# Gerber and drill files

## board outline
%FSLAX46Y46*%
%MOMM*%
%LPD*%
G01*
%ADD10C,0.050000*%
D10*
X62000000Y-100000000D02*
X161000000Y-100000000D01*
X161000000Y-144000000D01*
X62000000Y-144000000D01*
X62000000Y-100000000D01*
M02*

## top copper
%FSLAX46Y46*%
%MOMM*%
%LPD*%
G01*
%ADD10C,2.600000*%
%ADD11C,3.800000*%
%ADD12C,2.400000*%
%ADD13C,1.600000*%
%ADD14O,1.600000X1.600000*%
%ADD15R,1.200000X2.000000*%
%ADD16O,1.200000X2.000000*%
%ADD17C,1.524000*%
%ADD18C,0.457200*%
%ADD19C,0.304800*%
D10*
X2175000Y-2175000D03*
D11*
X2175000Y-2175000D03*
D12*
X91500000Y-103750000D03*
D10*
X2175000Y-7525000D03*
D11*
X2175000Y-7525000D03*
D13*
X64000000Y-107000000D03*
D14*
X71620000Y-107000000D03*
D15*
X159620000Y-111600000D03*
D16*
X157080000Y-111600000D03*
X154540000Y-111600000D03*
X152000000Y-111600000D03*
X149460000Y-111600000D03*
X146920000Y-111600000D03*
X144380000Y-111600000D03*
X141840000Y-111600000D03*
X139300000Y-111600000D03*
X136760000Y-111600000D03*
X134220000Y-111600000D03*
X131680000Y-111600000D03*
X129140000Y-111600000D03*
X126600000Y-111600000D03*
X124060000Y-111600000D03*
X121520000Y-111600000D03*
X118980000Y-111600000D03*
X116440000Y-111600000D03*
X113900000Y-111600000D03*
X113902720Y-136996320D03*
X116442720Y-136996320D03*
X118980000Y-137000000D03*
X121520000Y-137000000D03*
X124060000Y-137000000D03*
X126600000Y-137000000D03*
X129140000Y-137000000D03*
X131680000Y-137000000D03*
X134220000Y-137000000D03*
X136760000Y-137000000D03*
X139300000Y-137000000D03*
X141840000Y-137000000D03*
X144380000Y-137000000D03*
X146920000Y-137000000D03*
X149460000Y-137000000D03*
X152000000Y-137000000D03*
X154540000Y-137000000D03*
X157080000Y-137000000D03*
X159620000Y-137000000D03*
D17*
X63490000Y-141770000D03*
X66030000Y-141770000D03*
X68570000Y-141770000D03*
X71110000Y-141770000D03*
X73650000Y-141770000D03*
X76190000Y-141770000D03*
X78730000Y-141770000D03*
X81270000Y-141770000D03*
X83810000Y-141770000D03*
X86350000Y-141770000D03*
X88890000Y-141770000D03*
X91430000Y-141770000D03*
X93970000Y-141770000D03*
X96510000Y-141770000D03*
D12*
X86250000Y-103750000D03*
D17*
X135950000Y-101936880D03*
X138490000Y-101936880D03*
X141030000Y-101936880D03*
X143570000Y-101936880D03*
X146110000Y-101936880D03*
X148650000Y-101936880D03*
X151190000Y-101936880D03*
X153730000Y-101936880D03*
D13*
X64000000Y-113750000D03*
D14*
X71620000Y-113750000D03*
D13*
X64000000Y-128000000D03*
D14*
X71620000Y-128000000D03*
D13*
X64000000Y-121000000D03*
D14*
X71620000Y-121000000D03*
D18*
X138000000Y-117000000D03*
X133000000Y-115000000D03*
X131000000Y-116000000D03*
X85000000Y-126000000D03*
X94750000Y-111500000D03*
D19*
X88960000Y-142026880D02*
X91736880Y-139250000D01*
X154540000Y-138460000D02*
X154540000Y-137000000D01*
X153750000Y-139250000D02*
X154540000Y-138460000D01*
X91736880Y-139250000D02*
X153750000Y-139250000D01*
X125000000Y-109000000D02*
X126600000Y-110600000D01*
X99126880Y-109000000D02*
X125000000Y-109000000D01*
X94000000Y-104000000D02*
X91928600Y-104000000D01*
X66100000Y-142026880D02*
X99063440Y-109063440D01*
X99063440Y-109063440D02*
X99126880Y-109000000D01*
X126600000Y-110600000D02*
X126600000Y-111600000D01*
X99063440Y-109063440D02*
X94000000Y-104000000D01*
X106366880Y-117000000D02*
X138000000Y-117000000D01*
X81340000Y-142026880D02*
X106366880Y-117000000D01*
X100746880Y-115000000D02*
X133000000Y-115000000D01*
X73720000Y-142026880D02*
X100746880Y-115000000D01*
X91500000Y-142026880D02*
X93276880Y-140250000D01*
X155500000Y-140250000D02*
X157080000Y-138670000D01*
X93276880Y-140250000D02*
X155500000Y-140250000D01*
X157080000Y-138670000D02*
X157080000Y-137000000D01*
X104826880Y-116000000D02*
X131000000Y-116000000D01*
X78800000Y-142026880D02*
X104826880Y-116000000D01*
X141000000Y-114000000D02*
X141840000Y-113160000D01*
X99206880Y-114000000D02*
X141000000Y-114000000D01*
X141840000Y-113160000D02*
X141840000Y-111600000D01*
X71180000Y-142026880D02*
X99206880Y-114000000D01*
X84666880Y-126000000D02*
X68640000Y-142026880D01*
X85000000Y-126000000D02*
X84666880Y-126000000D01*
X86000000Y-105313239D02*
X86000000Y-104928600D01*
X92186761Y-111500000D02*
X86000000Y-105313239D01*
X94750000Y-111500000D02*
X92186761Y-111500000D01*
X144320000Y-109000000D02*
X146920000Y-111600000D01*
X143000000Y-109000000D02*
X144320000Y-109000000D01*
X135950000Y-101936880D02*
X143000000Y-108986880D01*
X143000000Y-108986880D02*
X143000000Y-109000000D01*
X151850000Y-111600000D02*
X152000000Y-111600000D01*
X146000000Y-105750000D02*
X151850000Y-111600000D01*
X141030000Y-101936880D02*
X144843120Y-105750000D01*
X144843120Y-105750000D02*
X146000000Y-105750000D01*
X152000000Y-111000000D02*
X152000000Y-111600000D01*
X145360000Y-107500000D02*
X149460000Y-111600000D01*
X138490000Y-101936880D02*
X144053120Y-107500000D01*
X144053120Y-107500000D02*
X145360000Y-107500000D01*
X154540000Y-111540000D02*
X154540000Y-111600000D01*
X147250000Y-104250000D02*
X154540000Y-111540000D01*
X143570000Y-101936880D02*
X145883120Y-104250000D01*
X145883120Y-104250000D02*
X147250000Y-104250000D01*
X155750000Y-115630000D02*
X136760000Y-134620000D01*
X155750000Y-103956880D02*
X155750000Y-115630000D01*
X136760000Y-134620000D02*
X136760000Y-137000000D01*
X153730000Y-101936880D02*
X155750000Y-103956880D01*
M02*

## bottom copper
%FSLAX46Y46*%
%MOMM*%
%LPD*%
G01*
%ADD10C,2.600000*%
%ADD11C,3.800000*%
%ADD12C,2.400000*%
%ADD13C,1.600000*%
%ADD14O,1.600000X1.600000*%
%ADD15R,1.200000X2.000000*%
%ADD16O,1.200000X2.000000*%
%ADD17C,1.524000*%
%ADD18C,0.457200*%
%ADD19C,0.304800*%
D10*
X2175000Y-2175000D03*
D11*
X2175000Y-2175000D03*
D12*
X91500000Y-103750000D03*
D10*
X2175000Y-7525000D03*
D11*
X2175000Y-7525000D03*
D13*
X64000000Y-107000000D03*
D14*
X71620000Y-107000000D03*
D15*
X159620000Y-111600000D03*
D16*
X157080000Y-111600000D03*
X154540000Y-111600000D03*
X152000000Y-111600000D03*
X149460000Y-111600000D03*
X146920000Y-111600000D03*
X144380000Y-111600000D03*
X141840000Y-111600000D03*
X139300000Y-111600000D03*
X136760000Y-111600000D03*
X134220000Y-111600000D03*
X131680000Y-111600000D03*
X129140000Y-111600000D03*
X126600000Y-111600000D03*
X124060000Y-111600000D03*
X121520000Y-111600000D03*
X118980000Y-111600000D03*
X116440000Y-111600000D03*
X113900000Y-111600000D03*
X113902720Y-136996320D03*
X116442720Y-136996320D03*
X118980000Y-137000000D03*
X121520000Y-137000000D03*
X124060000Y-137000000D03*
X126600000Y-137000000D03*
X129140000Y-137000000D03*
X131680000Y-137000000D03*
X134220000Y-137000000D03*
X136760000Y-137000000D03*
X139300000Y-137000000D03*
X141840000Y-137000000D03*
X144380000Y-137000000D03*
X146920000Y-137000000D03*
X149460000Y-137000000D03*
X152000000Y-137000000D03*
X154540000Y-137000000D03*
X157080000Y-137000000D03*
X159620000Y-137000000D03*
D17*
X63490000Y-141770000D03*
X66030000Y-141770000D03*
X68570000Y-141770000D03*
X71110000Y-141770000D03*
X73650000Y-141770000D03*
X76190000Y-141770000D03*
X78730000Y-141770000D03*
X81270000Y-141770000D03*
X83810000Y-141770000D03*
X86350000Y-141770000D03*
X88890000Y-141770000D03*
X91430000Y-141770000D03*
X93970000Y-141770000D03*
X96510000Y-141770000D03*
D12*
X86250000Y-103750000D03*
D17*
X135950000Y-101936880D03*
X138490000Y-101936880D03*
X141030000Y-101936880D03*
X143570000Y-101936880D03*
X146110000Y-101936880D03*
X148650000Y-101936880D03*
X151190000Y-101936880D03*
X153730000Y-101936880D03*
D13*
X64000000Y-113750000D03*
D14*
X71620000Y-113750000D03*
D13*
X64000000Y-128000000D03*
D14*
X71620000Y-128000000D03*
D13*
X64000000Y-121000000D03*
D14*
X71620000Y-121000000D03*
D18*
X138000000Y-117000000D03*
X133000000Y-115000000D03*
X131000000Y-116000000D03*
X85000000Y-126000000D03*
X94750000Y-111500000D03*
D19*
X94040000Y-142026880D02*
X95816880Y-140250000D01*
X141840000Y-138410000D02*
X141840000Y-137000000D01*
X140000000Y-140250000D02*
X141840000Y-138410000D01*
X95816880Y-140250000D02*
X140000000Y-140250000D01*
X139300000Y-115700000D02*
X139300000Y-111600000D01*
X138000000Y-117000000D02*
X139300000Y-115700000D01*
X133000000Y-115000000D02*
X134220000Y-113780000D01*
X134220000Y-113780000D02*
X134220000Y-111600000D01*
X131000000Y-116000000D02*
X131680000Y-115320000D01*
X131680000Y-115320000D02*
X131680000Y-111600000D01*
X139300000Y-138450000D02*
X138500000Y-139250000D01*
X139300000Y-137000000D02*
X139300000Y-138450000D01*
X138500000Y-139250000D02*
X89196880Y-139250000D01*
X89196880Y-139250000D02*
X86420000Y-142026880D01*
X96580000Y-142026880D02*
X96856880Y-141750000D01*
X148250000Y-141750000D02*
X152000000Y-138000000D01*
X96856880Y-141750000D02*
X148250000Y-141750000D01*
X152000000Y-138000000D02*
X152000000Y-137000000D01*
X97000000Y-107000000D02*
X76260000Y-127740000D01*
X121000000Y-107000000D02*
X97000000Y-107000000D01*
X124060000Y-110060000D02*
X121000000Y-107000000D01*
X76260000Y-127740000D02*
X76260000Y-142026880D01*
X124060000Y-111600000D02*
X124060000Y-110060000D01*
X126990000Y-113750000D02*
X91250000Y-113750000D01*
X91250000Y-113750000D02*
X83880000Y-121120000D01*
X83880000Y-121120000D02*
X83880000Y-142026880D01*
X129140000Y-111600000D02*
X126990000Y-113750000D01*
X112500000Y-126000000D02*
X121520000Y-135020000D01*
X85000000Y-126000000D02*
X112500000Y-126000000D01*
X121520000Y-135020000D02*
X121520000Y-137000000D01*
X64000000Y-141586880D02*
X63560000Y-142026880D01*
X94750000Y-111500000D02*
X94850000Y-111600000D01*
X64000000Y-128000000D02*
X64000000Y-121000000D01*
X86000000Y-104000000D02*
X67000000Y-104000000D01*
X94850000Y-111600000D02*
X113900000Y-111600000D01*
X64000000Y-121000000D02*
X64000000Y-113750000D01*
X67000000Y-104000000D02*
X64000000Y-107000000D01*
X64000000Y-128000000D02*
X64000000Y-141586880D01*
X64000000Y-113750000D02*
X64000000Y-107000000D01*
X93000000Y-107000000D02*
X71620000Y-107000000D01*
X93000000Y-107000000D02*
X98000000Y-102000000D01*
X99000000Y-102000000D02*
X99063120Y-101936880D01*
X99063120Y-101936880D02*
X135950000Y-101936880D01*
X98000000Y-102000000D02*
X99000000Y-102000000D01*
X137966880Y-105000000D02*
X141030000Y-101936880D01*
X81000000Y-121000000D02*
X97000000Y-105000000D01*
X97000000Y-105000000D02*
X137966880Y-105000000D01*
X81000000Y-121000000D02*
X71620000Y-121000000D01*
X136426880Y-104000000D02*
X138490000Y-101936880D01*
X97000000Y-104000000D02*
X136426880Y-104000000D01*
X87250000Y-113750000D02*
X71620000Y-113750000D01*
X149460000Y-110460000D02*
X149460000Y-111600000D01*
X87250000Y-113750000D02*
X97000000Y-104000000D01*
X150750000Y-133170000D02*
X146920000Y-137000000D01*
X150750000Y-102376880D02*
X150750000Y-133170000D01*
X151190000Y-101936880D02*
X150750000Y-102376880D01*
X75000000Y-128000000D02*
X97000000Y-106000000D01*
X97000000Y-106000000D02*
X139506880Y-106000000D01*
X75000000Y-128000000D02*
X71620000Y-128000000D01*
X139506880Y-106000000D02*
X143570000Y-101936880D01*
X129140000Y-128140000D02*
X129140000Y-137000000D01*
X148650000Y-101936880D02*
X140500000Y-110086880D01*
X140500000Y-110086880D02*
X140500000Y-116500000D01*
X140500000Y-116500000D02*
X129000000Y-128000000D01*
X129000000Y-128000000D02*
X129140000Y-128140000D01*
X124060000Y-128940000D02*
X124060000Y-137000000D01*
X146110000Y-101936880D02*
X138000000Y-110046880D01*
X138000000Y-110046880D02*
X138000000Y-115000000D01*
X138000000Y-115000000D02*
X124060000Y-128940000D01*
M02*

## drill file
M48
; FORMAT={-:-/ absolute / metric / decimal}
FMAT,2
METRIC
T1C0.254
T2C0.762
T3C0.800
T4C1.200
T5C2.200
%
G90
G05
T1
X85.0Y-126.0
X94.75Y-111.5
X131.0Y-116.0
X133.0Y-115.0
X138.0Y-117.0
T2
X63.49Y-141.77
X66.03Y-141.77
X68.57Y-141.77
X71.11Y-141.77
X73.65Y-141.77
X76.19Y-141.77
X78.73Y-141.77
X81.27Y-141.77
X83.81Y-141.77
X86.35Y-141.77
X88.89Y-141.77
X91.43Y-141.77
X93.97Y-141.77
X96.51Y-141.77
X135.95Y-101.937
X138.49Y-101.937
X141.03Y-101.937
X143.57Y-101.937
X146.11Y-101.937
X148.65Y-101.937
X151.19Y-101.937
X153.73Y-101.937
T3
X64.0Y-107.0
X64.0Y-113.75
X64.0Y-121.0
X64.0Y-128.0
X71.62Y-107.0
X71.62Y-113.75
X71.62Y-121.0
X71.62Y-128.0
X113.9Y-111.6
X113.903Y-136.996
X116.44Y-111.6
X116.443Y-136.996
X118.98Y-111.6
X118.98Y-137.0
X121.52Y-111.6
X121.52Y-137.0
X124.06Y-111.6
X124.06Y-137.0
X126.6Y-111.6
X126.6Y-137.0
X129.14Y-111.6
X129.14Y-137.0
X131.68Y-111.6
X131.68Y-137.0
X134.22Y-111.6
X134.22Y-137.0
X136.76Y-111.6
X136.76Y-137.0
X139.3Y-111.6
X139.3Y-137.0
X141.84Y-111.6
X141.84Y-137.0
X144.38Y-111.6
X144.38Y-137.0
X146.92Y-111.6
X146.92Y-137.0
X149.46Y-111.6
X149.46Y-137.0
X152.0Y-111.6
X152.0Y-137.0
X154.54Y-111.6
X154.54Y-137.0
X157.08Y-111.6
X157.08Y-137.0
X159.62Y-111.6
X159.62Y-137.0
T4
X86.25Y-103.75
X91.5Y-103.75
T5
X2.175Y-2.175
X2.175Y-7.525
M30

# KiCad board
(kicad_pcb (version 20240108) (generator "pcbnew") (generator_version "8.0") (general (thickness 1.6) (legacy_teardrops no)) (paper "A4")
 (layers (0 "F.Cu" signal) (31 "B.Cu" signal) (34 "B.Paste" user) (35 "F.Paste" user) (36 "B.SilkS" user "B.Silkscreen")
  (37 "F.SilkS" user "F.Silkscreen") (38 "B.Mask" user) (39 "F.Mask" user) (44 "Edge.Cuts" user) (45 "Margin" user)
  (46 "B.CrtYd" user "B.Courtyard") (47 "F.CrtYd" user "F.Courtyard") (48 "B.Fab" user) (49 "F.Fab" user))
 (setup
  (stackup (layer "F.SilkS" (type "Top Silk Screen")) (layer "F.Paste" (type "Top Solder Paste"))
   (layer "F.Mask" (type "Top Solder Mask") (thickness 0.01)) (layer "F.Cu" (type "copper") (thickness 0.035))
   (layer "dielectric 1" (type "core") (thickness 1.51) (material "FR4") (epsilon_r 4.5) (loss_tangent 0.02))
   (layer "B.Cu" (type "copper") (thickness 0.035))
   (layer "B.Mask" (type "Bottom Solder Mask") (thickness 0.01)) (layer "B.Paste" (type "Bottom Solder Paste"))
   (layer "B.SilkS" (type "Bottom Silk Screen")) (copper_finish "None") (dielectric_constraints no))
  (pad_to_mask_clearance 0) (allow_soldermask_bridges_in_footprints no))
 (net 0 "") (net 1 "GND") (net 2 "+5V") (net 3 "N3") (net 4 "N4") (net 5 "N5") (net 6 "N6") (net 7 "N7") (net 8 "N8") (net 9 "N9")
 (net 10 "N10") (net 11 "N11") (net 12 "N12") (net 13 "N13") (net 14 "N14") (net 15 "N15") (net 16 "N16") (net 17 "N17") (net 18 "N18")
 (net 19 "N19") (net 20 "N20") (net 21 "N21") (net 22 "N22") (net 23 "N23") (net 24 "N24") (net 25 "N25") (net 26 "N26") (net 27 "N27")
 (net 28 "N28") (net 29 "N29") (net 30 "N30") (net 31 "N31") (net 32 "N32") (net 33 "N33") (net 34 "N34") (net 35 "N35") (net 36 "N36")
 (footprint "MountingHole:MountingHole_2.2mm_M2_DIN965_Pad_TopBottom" (layer "F.Cu") (at 2.175 2.175)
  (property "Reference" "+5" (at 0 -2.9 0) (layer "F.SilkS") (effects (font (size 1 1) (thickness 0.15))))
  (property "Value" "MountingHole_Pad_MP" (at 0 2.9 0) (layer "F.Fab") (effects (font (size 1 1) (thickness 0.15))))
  (pad "1" thru_hole circle (at 0 0) (size 2.6 2.6) (drill 2.2) (layers "*.Cu" "*.Mask") (remove_unused_layers no))
  (pad "1" connect circle (at 0 0) (size 3.8 3.8) (layers "F.Cu" "F.Mask"))
  (pad "1" connect circle (at 0 0) (size 3.8 3.8) (layers "B.Cu" "B.Mask")))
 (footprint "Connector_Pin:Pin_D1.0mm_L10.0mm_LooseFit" (layer "F.Cu") (at 91.5 103.75)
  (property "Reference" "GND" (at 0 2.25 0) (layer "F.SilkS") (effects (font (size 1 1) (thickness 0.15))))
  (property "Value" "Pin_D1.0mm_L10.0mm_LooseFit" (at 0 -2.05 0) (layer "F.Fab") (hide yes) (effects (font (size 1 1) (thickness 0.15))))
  (pad "1" thru_hole circle (at 0 0) (size 2.4 2.4) (drill 1.2) (layers "*.Cu" "*.Mask") (remove_unused_layers no) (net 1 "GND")))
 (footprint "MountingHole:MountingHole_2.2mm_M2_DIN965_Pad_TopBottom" (layer "F.Cu") (at 2.175 7.525)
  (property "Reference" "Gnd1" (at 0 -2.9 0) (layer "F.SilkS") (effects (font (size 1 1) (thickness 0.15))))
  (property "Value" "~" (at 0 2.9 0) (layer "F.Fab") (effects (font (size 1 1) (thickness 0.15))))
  (pad "1" thru_hole circle (at 0 0) (size 2.6 2.6) (drill 2.2) (layers "*.Cu" "*.Mask") (remove_unused_layers no))
  (pad "1" connect circle (at 0 0) (size 3.8 3.8) (layers "F.Cu" "F.Mask"))
  (pad "1" connect circle (at 0 0) (size 3.8 3.8) (layers "B.Cu" "B.Mask")))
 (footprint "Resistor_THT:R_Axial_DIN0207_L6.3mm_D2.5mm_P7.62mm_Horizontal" (layer "F.Cu") (at 64 107)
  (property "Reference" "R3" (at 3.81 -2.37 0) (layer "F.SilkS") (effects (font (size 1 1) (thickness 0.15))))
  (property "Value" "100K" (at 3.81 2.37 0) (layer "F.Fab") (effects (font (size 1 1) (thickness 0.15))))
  (pad "1" thru_hole circle (at 0 0) (size 1.6 1.6) (drill 0.8) (layers "*.Cu" "*.Mask") (remove_unused_layers no) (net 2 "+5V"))
  (pad "2" thru_hole oval (at 7.62 0) (size 1.6 1.6) (drill 0.8) (layers "*.Cu" "*.Mask") (remove_unused_layers no) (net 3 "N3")))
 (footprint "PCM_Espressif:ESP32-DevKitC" (layer "F.Cu") (at 159.62 111.6 -90)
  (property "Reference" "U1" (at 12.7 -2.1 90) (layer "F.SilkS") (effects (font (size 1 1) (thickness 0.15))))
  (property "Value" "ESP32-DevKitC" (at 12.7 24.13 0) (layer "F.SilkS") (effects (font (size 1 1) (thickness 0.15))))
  (pad "1" thru_hole rect (at 0 0 180) (size 1.2 2) (drill 0.8) (layers "*.Cu" "*.Mask") (remove_unused_layers no) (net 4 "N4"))
  (pad "2" thru_hole oval (at 0 2.54 180) (size 1.2 2) (drill 0.8) (layers "*.Cu" "*.Mask") (remove_unused_layers no) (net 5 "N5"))
  (pad "3" thru_hole oval (at 0 5.08 180) (size 1.2 2) (drill 0.8) (layers "*.Cu" "*.Mask") (remove_unused_layers no) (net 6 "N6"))
  (pad "4" thru_hole oval (at 0 7.62 180) (size 1.2 2) (drill 0.8) (layers "*.Cu" "*.Mask") (remove_unused_layers no) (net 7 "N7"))
  (pad "5" thru_hole oval (at 0 10.16 180) (size 1.2 2) (drill 0.8) (layers "*.Cu" "*.Mask") (remove_unused_layers no) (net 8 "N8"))
  (pad "6" thru_hole oval (at 0 12.7 180) (size 1.2 2) (drill 0.8) (layers "*.Cu" "*.Mask") (remove_unused_layers no) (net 3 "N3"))
  (pad "7" thru_hole oval (at 0 15.24 180) (size 1.2 2) (drill 0.8) (layers "*.Cu" "*.Mask") (remove_unused_layers no) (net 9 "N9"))
  (pad "8" thru_hole oval (at 0 17.78 180) (size 1.2 2) (drill 0.8) (layers "*.Cu" "*.Mask") (remove_unused_layers no) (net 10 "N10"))
  (pad "9" thru_hole oval (at 0 20.32 180) (size 1.2 2) (drill 0.8) (layers "*.Cu" "*.Mask") (remove_unused_layers no) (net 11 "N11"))
  (pad "10" thru_hole oval (at 0 22.86 180) (size 1.2 2) (drill 0.8) (layers "*.Cu" "*.Mask") (remove_unused_layers no) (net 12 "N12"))
  (pad "11" thru_hole oval (at 0 25.4 180) (size 1.2 2) (drill 0.8) (layers "*.Cu" "*.Mask") (remove_unused_layers no) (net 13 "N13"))
  (pad "12" thru_hole oval (at 0 27.94 180) (size 1.2 2) (drill 0.8) (layers "*.Cu" "*.Mask") (remove_unused_layers no) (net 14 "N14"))
  (pad "13" thru_hole oval (at 0 30.48 180) (size 1.2 2) (drill 0.8) (layers "*.Cu" "*.Mask") (remove_unused_layers no) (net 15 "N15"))
  (pad "14" thru_hole oval (at 0 33.02 180) (size 1.2 2) (drill 0.8) (layers "*.Cu" "*.Mask") (remove_unused_layers no) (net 1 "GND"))
  (pad "15" thru_hole oval (at 0 35.56 180) (size 1.2 2) (drill 0.8) (layers "*.Cu" "*.Mask") (remove_unused_layers no) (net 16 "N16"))
  (pad "16" thru_hole oval (at 0 38.1 180) (size 1.2 2) (drill 0.8) (layers "*.Cu" "*.Mask") (remove_unused_layers no) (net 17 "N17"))
  (pad "17" thru_hole oval (at 0 40.64 180) (size 1.2 2) (drill 0.8) (layers "*.Cu" "*.Mask") (remove_unused_layers no) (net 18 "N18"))
  (pad "18" thru_hole oval (at 0 43.18 180) (size 1.2 2) (drill 0.8) (layers "*.Cu" "*.Mask") (remove_unused_layers no) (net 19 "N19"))
  (pad "19" thru_hole oval (at 0 45.72 180) (size 1.2 2) (drill 0.8) (layers "*.Cu" "*.Mask") (remove_unused_layers no) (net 2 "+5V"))
  (pad "20" thru_hole oval (at 25.39632 45.71728 180) (size 1.2 2) (drill 0.8) (layers "*.Cu" "*.Mask") (remove_unused_layers no)
   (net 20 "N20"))
  (pad "21" thru_hole oval (at 25.39632 43.17728 180) (size 1.2 2) (drill 0.8) (layers "*.Cu" "*.Mask") (remove_unused_layers no)
   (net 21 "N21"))
  (pad "22" thru_hole oval (at 25.4 40.64 180) (size 1.2 2) (drill 0.8) (layers "*.Cu" "*.Mask") (remove_unused_layers no) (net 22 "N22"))
  (pad "23" thru_hole oval (at 25.4 38.1 180) (size 1.2 2) (drill 0.8) (layers "*.Cu" "*.Mask") (remove_unused_layers no) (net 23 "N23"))
  (pad "24" thru_hole oval (at 25.4 35.56 180) (size 1.2 2) (drill 0.8) (layers "*.Cu" "*.Mask") (remove_unused_layers no) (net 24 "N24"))
  (pad "25" thru_hole oval (at 25.4 33.02 180) (size 1.2 2) (drill 0.8) (layers "*.Cu" "*.Mask") (remove_unused_layers no) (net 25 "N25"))
  (pad "26" thru_hole oval (at 25.4 30.48 180) (size 1.2 2) (drill 0.8) (layers "*.Cu" "*.Mask") (remove_unused_layers no) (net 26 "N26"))
  (pad "27" thru_hole oval (at 25.4 27.94 180) (size 1.2 2) (drill 0.8) (layers "*.Cu" "*.Mask") (remove_unused_layers no) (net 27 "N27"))
  (pad "28" thru_hole oval (at 25.4 25.4 180) (size 1.2 2) (drill 0.8) (layers "*.Cu" "*.Mask") (remove_unused_layers no) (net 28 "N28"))
  (pad "29" thru_hole oval (at 25.4 22.86 180) (size 1.2 2) (drill 0.8) (layers "*.Cu" "*.Mask") (remove_unused_layers no) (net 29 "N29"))
  (pad "30" thru_hole oval (at 25.4 20.32 180) (size 1.2 2) (drill 0.8) (layers "*.Cu" "*.Mask") (remove_unused_layers no) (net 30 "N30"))
  (pad "31" thru_hole oval (at 25.4 17.78 180) (size 1.2 2) (drill 0.8) (layers "*.Cu" "*.Mask") (remove_unused_layers no) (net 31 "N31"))
  (pad "32" thru_hole oval (at 25.4 15.24 180) (size 1.2 2) (drill 0.8) (layers "*.Cu" "*.Mask") (remove_unused_layers no) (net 1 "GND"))
  (pad "33" thru_hole oval (at 25.4 12.7 180) (size 1.2 2) (drill 0.8) (layers "*.Cu" "*.Mask") (remove_unused_layers no) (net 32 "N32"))
  (pad "34" thru_hole oval (at 25.4 10.16 180) (size 1.2 2) (drill 0.8) (layers "*.Cu" "*.Mask") (remove_unused_layers no) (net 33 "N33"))
  (pad "35" thru_hole oval (at 25.4 7.62 180) (size 1.2 2) (drill 0.8) (layers "*.Cu" "*.Mask") (remove_unused_layers no) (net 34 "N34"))
  (pad "36" thru_hole oval (at 25.4 5.08 180) (size 1.2 2) (drill 0.8) (layers "*.Cu" "*.Mask") (remove_unused_layers no) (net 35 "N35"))
  (pad "37" thru_hole oval (at 25.4 2.54 180) (size 1.2 2) (drill 0.8) (layers "*.Cu" "*.Mask") (remove_unused_layers no) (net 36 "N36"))
  (pad "38" thru_hole oval (at 25.4 0 180) (size 1.2 2) (drill 0.8) (layers "*.Cu" "*.Mask") (remove_unused_layers no) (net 1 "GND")))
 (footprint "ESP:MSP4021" (layer "F.Cu") (at 63.49 141.77)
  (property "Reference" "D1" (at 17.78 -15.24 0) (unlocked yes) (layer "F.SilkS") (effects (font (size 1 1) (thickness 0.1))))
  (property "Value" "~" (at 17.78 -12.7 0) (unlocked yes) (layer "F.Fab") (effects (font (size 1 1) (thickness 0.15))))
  (pad "1" thru_hole circle (at 0 0) (size 1.524 1.524) (drill 0.762) (layers "*.Cu" "*.Mask") (remove_unused_layers no) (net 2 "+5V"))
  (pad "2" thru_hole circle (at 2.54 0) (size 1.524 1.524) (drill 0.762) (layers "*.Cu" "*.Mask") (remove_unused_layers no) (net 1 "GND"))
  (pad "3" thru_hole circle (at 5.08 0) (size 1.524 1.524) (drill 0.762) (layers "*.Cu" "*.Mask") (remove_unused_layers no) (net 23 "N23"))
  (pad "4" thru_hole circle (at 7.62 0) (size 1.524 1.524) (drill 0.762) (layers "*.Cu" "*.Mask") (remove_unused_layers no) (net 10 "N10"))
  (pad "5" thru_hole circle (at 10.16 0) (size 1.524 1.524) (drill 0.762) (layers "*.Cu" "*.Mask") (remove_unused_layers no) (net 13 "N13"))
  (pad "6" thru_hole circle (at 12.7 0) (size 1.524 1.524) (drill 0.762) (layers "*.Cu" "*.Mask") (remove_unused_layers no) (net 16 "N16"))
  (pad "7" thru_hole circle (at 15.24 0) (size 1.524 1.524) (drill 0.762) (layers "*.Cu" "*.Mask") (remove_unused_layers no) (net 14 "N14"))
  (pad "8" thru_hole circle (at 17.78 0) (size 1.524 1.524) (drill 0.762) (layers "*.Cu" "*.Mask") (remove_unused_layers no) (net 11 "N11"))
  (pad "9" thru_hole circle (at 20.32 0) (size 1.524 1.524) (drill 0.762) (layers "*.Cu" "*.Mask") (remove_unused_layers no) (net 15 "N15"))
  (pad "10" thru_hole circle (at 22.86 0) (size 1.524 1.524) (drill 0.762) (layers "*.Cu" "*.Mask") (remove_unused_layers no) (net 30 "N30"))
  (pad "11" thru_hole circle (at 25.4 0) (size 1.524 1.524) (drill 0.762) (layers "*.Cu" "*.Mask") (remove_unused_layers no) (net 35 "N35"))
  (pad "12" thru_hole circle (at 27.94 0) (size 1.524 1.524) (drill 0.762) (layers "*.Cu" "*.Mask") (remove_unused_layers no) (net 36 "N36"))
  (pad "13" thru_hole circle (at 30.48 0) (size 1.524 1.524) (drill 0.762) (layers "*.Cu" "*.Mask") (remove_unused_layers no) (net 31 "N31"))
  (pad "14" thru_hole circle (at 33.02 0) (size 1.524 1.524) (drill 0.762) (layers "*.Cu" "*.Mask") (remove_unused_layers no) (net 34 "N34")))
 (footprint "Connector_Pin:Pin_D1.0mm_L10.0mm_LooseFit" (layer "F.Cu") (at 86.25 103.75)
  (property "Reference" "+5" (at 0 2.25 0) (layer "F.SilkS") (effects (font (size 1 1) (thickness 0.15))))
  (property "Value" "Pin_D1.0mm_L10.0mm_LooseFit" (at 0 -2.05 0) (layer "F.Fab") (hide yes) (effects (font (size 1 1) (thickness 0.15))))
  (pad "1" thru_hole circle (at 0 0) (size 2.4 2.4) (drill 1.2) (layers "*.Cu" "*.Mask") (remove_unused_layers no) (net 2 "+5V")))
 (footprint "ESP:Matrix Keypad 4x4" (layer "F.Cu") (at 135.95 101.93688)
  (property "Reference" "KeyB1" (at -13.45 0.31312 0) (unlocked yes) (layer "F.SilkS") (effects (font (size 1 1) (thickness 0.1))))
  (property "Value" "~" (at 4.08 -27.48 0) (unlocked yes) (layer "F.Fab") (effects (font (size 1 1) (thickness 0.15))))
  (pad "1" thru_hole circle (at 0 0) (size 1.524 1.524) (drill 0.762) (layers "*.Cu" "*.Mask") (remove_unused_layers no) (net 3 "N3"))
  (pad "2" thru_hole circle (at 2.54 0) (size 1.524 1.524) (drill 0.762) (layers "*.Cu" "*.Mask") (remove_unused_layers no) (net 8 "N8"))
  (pad "3" thru_hole circle (at 5.08 0) (size 1.524 1.524) (drill 0.762) (layers "*.Cu" "*.Mask") (remove_unused_layers no) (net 7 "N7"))
  (pad "4" thru_hole circle (at 7.62 0) (size 1.524 1.524) (drill 0.762) (layers "*.Cu" "*.Mask") (remove_unused_layers no) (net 6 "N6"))
  (pad "5" thru_hole circle (at 10.16 0) (size 1.524 1.524) (drill 0.762) (layers "*.Cu" "*.Mask") (remove_unused_layers no) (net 24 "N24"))
  (pad "6" thru_hole circle (at 12.7 0) (size 1.524 1.524) (drill 0.762) (layers "*.Cu" "*.Mask") (remove_unused_layers no) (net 26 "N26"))
  (pad "7" thru_hole circle (at 15.24 0) (size 1.524 1.524) (drill 0.762) (layers "*.Cu" "*.Mask") (remove_unused_layers no) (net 32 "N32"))
  (pad "8" thru_hole circle (at 17.78 0) (size 1.524 1.524) (drill 0.762) (layers "*.Cu" "*.Mask") (remove_unused_layers no) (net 29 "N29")))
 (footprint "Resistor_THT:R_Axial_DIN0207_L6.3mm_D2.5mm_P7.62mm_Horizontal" (layer "F.Cu") (at 64 113.75)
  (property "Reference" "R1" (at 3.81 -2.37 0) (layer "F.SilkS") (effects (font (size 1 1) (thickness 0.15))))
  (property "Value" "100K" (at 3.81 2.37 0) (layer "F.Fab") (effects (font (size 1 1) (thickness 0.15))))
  (pad "1" thru_hole circle (at 0 0) (size 1.6 1.6) (drill 0.8) (layers "*.Cu" "*.Mask") (remove_unused_layers no) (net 2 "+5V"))
  (pad "2" thru_hole oval (at 7.62 0) (size 1.6 1.6) (drill 0.8) (layers "*.Cu" "*.Mask") (remove_unused_layers no) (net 7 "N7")))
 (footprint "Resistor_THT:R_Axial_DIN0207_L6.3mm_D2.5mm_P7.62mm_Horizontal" (layer "F.Cu") (at 64 128)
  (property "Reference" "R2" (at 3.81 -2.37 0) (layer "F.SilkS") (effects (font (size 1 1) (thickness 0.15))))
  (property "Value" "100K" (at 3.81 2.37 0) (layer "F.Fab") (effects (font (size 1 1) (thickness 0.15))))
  (pad "1" thru_hole circle (at 0 0) (size 1.6 1.6) (drill 0.8) (layers "*.Cu" "*.Mask") (remove_unused_layers no) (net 2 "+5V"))
  (pad "2" thru_hole oval (at 7.62 0) (size 1.6 1.6) (drill 0.8) (layers "*.Cu" "*.Mask") (remove_unused_layers no) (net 6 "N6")))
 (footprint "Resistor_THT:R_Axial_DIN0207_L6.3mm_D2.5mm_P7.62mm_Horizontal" (layer "F.Cu") (at 64 121)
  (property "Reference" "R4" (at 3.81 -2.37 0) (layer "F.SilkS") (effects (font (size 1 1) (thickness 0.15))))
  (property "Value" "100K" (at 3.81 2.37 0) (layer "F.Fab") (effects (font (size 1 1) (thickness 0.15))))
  (pad "1" thru_hole circle (at 0 0) (size 1.6 1.6) (drill 0.8) (layers "*.Cu" "*.Mask") (remove_unused_layers no) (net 2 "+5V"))
  (pad "2" thru_hole oval (at 7.62 0) (size 1.6 1.6) (drill 0.8) (layers "*.Cu" "*.Mask") (remove_unused_layers no) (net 8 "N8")))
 (gr_rect (start 62 100) (end 161 144) (stroke (width 0.05) (type default)) (fill none) (layer "Edge.Cuts"))
 (segment (start 88.96 142.02688) (end 91.73688 139.25) (width 0.3048) (layer "F.Cu") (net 35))
 (segment (start 154.54 138.46) (end 154.54 137) (width 0.3048) (layer "F.Cu") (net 35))
 (segment (start 153.75 139.25) (end 154.54 138.46) (width 0.3048) (layer "F.Cu") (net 35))
 (segment (start 91.73688 139.25) (end 153.75 139.25) (width 0.3048) (layer "F.Cu") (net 35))
 (segment (start 94.04 142.02688) (end 95.81688 140.25) (width 0.3048) (layer "B.Cu") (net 31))
 (segment (start 141.84 138.41) (end 141.84 137) (width 0.3048) (layer "B.Cu") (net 31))
 (segment (start 140 140.25) (end 141.84 138.41) (width 0.3048) (layer "B.Cu") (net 31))
 (segment (start 95.81688 140.25) (end 140 140.25) (width 0.3048) (layer "B.Cu") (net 31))
 (segment (start 125 109) (end 126.6 110.6) (width 0.3048) (layer "F.Cu") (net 1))
 (segment (start 99.12688 109) (end 125 109) (width 0.3048) (layer "F.Cu") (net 1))
 (segment (start 94 104) (end 91.9286 104) (width 0.3048) (layer "F.Cu") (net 1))
 (segment (start 66.1 142.02688) (end 99.06344 109.06344) (width 0.3048) (layer "F.Cu") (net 1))
 (segment (start 99.06344 109.06344) (end 99.12688 109) (width 0.3048) (layer "F.Cu") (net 1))
 (segment (start 126.6 110.6) (end 126.6 111.6) (width 0.3048) (layer "F.Cu") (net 1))
 (segment (start 99.06344 109.06344) (end 94 104) (width 0.3048) (layer "F.Cu") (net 1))
 (segment (start 106.36688 117) (end 138 117) (width 0.3048) (layer "F.Cu") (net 11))
 (segment (start 81.34 142.02688) (end 106.36688 117) (width 0.3048) (layer "F.Cu") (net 11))
 (via (at 138 117) (size 0.4572) (drill 0.254) (layers "F.Cu" "B.Cu") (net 11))
 (segment (start 139.3 115.7) (end 139.3 111.6) (width 0.3048) (layer "B.Cu") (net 11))
 (segment (start 138 117) (end 139.3 115.7) (width 0.3048) (layer "B.Cu") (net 11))
 (segment (start 100.74688 115) (end 133 115) (width 0.3048) (layer "F.Cu") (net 13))
 (segment (start 73.72 142.02688) (end 100.74688 115) (width 0.3048) (layer "F.Cu") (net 13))
 (via (at 133 115) (size 0.4572) (drill 0.254) (layers "F.Cu" "B.Cu") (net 13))
 (segment (start 133 115) (end 134.22 113.78) (width 0.3048) (layer "B.Cu") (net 13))
 (segment (start 134.22 113.78) (end 134.22 111.6) (width 0.3048) (layer "B.Cu") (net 13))
 (segment (start 91.5 142.02688) (end 93.27688 140.25) (width 0.3048) (layer "F.Cu") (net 36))
 (segment (start 155.5 140.25) (end 157.08 138.67) (width 0.3048) (layer "F.Cu") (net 36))
 (segment (start 93.27688 140.25) (end 155.5 140.25) (width 0.3048) (layer "F.Cu") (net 36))
 (segment (start 157.08 138.67) (end 157.08 137) (width 0.3048) (layer "F.Cu") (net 36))
 (segment (start 104.82688 116) (end 131 116) (width 0.3048) (layer "F.Cu") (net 14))
 (segment (start 78.8 142.02688) (end 104.82688 116) (width 0.3048) (layer "F.Cu") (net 14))
 (via (at 131 116) (size 0.4572) (drill 0.254) (layers "F.Cu" "B.Cu") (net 14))
 (segment (start 131 116) (end 131.68 115.32) (width 0.3048) (layer "B.Cu") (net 14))
 (segment (start 131.68 115.32) (end 131.68 111.6) (width 0.3048) (layer "B.Cu") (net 14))
 (segment (start 139.3 138.45) (end 138.5 139.25) (width 0.3048) (layer "B.Cu") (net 30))
 (segment (start 139.3 137) (end 139.3 138.45) (width 0.3048) (layer "B.Cu") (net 30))
 (segment (start 138.5 139.25) (end 89.19688 139.25) (width 0.3048) (layer "B.Cu") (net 30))
 (segment (start 89.19688 139.25) (end 86.42 142.02688) (width 0.3048) (layer "B.Cu") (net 30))
 (segment (start 96.58 142.02688) (end 96.85688 141.75) (width 0.3048) (layer "B.Cu") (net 34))
 (segment (start 148.25 141.75) (end 152 138) (width 0.3048) (layer "B.Cu") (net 34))
 (segment (start 96.85688 141.75) (end 148.25 141.75) (width 0.3048) (layer "B.Cu") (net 34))
 (segment (start 152 138) (end 152 137) (width 0.3048) (layer "B.Cu") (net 34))
 (segment (start 141 114) (end 141.84 113.16) (width 0.3048) (layer "F.Cu") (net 10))
 (segment (start 99.20688 114) (end 141 114) (width 0.3048) (layer "F.Cu") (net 10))
 (segment (start 141.84 113.16) (end 141.84 111.6) (width 0.3048) (layer "F.Cu") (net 10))
 (segment (start 71.18 142.02688) (end 99.20688 114) (width 0.3048) (layer "F.Cu") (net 10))
 (segment (start 97 107) (end 76.26 127.74) (width 0.3048) (layer "B.Cu") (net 16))
 (segment (start 121 107) (end 97 107) (width 0.3048) (layer "B.Cu") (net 16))
 (segment (start 124.06 110.06) (end 121 107) (width 0.3048) (layer "B.Cu") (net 16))
 (segment (start 76.26 127.74) (end 76.26 142.02688) (width 0.3048) (layer "B.Cu") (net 16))
 (segment (start 124.06 111.6) (end 124.06 110.06) (width 0.3048) (layer "B.Cu") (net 16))
 (segment (start 126.99 113.75) (end 91.25 113.75) (width 0.3048) (layer "B.Cu") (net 15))
 (segment (start 91.25 113.75) (end 83.88 121.12) (width 0.3048) (layer "B.Cu") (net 15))
 (segment (start 83.88 121.12) (end 83.88 142.02688) (width 0.3048) (layer "B.Cu") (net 15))
 (segment (start 129.14 111.6) (end 126.99 113.75) (width 0.3048) (layer "B.Cu") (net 15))
 (segment (start 84.66688 126) (end 68.64 142.02688) (width 0.3048) (layer "F.Cu") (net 23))
 (segment (start 85 126) (end 84.66688 126) (width 0.3048) (layer "F.Cu") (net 23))
 (via (at 85 126) (size 0.4572) (drill 0.254) (layers "F.Cu" "B.Cu") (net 23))
 (segment (start 112.5 126) (end 121.52 135.02) (width 0.3048) (layer "B.Cu") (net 23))
 (segment (start 85 126) (end 112.5 126) (width 0.3048) (layer "B.Cu") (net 23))
 (segment (start 121.52 135.02) (end 121.52 137) (width 0.3048) (layer "B.Cu") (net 23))
 (segment (start 86 105.313239) (end 86 104.9286) (width 0.3048) (layer "F.Cu") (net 2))
 (segment (start 92.186761 111.5) (end 86 105.313239) (width 0.3048) (layer "F.Cu") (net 2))
 (segment (start 94.75 111.5) (end 92.186761 111.5) (width 0.3048) (layer "F.Cu") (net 2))
 (via (at 94.75 111.5) (size 0.4572) (drill 0.254) (layers "F.Cu" "B.Cu") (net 2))
 (segment (start 64 141.58688) (end 63.56 142.02688) (width 0.3048) (layer "B.Cu") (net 2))
 (segment (start 94.75 111.5) (end 94.85 111.6) (width 0.3048) (layer "B.Cu") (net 2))
 (segment (start 64 128) (end 64 121) (width 0.3048) (layer "B.Cu") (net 2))
 (segment (start 86 104) (end 67 104) (width 0.3048) (layer "B.Cu") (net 2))
 (segment (start 94.85 111.6) (end 113.9 111.6) (width 0.3048) (layer "B.Cu") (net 2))
 (segment (start 64 121) (end 64 113.75) (width 0.3048) (layer "B.Cu") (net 2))
 (segment (start 67 104) (end 64 107) (width 0.3048) (layer "B.Cu") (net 2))
 (segment (start 64 128) (end 64 141.58688) (width 0.3048) (layer "B.Cu") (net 2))
 (segment (start 64 113.75) (end 64 107) (width 0.3048) (layer "B.Cu") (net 2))
 (segment (start 144.32 109) (end 146.92 111.6) (width 0.3048) (layer "F.Cu") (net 3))
 (segment (start 143 109) (end 144.32 109) (width 0.3048) (layer "F.Cu") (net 3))
 (segment (start 135.95 101.93688) (end 143 108.98688) (width 0.3048) (layer "F.Cu") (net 3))
 (segment (start 143 108.98688) (end 143 109) (width 0.3048) (layer "F.Cu") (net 3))
 (segment (start 93 107) (end 71.62 107) (width 0.3048) (layer "B.Cu") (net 3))
 (segment (start 93 107) (end 98 102) (width 0.3048) (layer "B.Cu") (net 3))
 (segment (start 99 102) (end 99.06312 101.93688) (width 0.3048) (layer "B.Cu") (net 3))
 (segment (start 99.06312 101.93688) (end 135.95 101.93688) (width 0.3048) (layer "B.Cu") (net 3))
 (segment (start 98 102) (end 99 102) (width 0.3048) (layer "B.Cu") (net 3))
 (segment (start 151.85 111.6) (end 152 111.6) (width 0.3048) (layer "F.Cu") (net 7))
 (segment (start 146 105.75) (end 151.85 111.6) (width 0.3048) (layer "F.Cu") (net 7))
 (segment (start 141.03 101.93688) (end 144.84312 105.75) (width 0.3048) (layer "F.Cu") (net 7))
 (segment (start 144.84312 105.75) (end 146 105.75) (width 0.3048) (layer "F.Cu") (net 7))
 (segment (start 152 111) (end 152 111.6) (width 0.3048) (layer "F.Cu") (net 7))
 (segment (start 137.96688 105) (end 141.03 101.93688) (width 0.3048) (layer "B.Cu") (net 7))
 (segment (start 81 121) (end 97 105) (width 0.3048) (layer "B.Cu") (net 7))
 (segment (start 97 105) (end 137.96688 105) (width 0.3048) (layer "B.Cu") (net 7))
 (segment (start 81 121) (end 71.62 121) (width 0.3048) (layer "B.Cu") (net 7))
 (segment (start 145.36 107.5) (end 149.46 111.6) (width 0.3048) (layer "F.Cu") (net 8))
 (segment (start 138.49 101.93688) (end 144.05312 107.5) (width 0.3048) (layer "F.Cu") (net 8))
 (segment (start 144.05312 107.5) (end 145.36 107.5) (width 0.3048) (layer "F.Cu") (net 8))
 (segment (start 136.42688 104) (end 138.49 101.93688) (width 0.3048) (layer "B.Cu") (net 8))
 (segment (start 97 104) (end 136.42688 104) (width 0.3048) (layer "B.Cu") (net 8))
 (segment (start 87.25 113.75) (end 71.62 113.75) (width 0.3048) (layer "B.Cu") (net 8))
 (segment (start 149.46 110.46) (end 149.46 111.6) (width 0.3048) (layer "B.Cu") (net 8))
 (segment (start 87.25 113.75) (end 97 104) (width 0.3048) (layer "B.Cu") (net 8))
 (segment (start 150.75 133.17) (end 146.92 137) (width 0.3048) (layer "B.Cu") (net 32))
 (segment (start 150.75 102.37688) (end 150.75 133.17) (width 0.3048) (layer "B.Cu") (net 32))
 (segment (start 151.19 101.93688) (end 150.75 102.37688) (width 0.3048) (layer "B.Cu") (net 32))
 (segment (start 154.54 111.54) (end 154.54 111.6) (width 0.3048) (layer "F.Cu") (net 6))
 (segment (start 147.25 104.25) (end 154.54 111.54) (width 0.3048) (layer "F.Cu") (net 6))
 (segment (start 143.57 101.93688) (end 145.88312 104.25) (width 0.3048) (layer "F.Cu") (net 6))
 (segment (start 145.88312 104.25) (end 147.25 104.25) (width 0.3048) (layer "F.Cu") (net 6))
 (segment (start 75 128) (end 97 106) (width 0.3048) (layer "B.Cu") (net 6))
 (segment (start 97 106) (end 139.50688 106) (width 0.3048) (layer "B.Cu") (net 6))
 (segment (start 75 128) (end 71.62 128) (width 0.3048) (layer "B.Cu") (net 6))
 (segment (start 139.50688 106) (end 143.57 101.93688) (width 0.3048) (layer "B.Cu") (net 6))
 (segment (start 129.14 128.14) (end 129.14 137) (width 0.3048) (layer "B.Cu") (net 26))
 (segment (start 148.65 101.93688) (end 140.5 110.08688) (width 0.3048) (layer "B.Cu") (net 26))
 (segment (start 140.5 110.08688) (end 140.5 116.5) (width 0.3048) (layer "B.Cu") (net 26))
 (segment (start 140.5 116.5) (end 129 128) (width 0.3048) (layer "B.Cu") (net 26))
 (segment (start 129 128) (end 129.14 128.14) (width 0.3048) (layer "B.Cu") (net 26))
 (segment (start 124.06 128.94) (end 124.06 137) (width 0.3048) (layer "B.Cu") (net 24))
 (segment (start 146.11 101.93688) (end 138 110.04688) (width 0.3048) (layer "B.Cu") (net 24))
 (segment (start 138 110.04688) (end 138 115) (width 0.3048) (layer "B.Cu") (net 24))
 (segment (start 138 115) (end 124.06 128.94) (width 0.3048) (layer "B.Cu") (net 24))
 (segment (start 155.75 115.63) (end 136.76 134.62) (width 0.3048) (layer "F.Cu") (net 29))
 (segment (start 155.75 103.95688) (end 155.75 115.63) (width 0.3048) (layer "F.Cu") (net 29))
 (segment (start 136.76 134.62) (end 136.76 137) (width 0.3048) (layer "F.Cu") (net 29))
 (segment (start 153.73 101.93688) (end 155.75 103.95688) (width 0.3048) (layer "F.Cu") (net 29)))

